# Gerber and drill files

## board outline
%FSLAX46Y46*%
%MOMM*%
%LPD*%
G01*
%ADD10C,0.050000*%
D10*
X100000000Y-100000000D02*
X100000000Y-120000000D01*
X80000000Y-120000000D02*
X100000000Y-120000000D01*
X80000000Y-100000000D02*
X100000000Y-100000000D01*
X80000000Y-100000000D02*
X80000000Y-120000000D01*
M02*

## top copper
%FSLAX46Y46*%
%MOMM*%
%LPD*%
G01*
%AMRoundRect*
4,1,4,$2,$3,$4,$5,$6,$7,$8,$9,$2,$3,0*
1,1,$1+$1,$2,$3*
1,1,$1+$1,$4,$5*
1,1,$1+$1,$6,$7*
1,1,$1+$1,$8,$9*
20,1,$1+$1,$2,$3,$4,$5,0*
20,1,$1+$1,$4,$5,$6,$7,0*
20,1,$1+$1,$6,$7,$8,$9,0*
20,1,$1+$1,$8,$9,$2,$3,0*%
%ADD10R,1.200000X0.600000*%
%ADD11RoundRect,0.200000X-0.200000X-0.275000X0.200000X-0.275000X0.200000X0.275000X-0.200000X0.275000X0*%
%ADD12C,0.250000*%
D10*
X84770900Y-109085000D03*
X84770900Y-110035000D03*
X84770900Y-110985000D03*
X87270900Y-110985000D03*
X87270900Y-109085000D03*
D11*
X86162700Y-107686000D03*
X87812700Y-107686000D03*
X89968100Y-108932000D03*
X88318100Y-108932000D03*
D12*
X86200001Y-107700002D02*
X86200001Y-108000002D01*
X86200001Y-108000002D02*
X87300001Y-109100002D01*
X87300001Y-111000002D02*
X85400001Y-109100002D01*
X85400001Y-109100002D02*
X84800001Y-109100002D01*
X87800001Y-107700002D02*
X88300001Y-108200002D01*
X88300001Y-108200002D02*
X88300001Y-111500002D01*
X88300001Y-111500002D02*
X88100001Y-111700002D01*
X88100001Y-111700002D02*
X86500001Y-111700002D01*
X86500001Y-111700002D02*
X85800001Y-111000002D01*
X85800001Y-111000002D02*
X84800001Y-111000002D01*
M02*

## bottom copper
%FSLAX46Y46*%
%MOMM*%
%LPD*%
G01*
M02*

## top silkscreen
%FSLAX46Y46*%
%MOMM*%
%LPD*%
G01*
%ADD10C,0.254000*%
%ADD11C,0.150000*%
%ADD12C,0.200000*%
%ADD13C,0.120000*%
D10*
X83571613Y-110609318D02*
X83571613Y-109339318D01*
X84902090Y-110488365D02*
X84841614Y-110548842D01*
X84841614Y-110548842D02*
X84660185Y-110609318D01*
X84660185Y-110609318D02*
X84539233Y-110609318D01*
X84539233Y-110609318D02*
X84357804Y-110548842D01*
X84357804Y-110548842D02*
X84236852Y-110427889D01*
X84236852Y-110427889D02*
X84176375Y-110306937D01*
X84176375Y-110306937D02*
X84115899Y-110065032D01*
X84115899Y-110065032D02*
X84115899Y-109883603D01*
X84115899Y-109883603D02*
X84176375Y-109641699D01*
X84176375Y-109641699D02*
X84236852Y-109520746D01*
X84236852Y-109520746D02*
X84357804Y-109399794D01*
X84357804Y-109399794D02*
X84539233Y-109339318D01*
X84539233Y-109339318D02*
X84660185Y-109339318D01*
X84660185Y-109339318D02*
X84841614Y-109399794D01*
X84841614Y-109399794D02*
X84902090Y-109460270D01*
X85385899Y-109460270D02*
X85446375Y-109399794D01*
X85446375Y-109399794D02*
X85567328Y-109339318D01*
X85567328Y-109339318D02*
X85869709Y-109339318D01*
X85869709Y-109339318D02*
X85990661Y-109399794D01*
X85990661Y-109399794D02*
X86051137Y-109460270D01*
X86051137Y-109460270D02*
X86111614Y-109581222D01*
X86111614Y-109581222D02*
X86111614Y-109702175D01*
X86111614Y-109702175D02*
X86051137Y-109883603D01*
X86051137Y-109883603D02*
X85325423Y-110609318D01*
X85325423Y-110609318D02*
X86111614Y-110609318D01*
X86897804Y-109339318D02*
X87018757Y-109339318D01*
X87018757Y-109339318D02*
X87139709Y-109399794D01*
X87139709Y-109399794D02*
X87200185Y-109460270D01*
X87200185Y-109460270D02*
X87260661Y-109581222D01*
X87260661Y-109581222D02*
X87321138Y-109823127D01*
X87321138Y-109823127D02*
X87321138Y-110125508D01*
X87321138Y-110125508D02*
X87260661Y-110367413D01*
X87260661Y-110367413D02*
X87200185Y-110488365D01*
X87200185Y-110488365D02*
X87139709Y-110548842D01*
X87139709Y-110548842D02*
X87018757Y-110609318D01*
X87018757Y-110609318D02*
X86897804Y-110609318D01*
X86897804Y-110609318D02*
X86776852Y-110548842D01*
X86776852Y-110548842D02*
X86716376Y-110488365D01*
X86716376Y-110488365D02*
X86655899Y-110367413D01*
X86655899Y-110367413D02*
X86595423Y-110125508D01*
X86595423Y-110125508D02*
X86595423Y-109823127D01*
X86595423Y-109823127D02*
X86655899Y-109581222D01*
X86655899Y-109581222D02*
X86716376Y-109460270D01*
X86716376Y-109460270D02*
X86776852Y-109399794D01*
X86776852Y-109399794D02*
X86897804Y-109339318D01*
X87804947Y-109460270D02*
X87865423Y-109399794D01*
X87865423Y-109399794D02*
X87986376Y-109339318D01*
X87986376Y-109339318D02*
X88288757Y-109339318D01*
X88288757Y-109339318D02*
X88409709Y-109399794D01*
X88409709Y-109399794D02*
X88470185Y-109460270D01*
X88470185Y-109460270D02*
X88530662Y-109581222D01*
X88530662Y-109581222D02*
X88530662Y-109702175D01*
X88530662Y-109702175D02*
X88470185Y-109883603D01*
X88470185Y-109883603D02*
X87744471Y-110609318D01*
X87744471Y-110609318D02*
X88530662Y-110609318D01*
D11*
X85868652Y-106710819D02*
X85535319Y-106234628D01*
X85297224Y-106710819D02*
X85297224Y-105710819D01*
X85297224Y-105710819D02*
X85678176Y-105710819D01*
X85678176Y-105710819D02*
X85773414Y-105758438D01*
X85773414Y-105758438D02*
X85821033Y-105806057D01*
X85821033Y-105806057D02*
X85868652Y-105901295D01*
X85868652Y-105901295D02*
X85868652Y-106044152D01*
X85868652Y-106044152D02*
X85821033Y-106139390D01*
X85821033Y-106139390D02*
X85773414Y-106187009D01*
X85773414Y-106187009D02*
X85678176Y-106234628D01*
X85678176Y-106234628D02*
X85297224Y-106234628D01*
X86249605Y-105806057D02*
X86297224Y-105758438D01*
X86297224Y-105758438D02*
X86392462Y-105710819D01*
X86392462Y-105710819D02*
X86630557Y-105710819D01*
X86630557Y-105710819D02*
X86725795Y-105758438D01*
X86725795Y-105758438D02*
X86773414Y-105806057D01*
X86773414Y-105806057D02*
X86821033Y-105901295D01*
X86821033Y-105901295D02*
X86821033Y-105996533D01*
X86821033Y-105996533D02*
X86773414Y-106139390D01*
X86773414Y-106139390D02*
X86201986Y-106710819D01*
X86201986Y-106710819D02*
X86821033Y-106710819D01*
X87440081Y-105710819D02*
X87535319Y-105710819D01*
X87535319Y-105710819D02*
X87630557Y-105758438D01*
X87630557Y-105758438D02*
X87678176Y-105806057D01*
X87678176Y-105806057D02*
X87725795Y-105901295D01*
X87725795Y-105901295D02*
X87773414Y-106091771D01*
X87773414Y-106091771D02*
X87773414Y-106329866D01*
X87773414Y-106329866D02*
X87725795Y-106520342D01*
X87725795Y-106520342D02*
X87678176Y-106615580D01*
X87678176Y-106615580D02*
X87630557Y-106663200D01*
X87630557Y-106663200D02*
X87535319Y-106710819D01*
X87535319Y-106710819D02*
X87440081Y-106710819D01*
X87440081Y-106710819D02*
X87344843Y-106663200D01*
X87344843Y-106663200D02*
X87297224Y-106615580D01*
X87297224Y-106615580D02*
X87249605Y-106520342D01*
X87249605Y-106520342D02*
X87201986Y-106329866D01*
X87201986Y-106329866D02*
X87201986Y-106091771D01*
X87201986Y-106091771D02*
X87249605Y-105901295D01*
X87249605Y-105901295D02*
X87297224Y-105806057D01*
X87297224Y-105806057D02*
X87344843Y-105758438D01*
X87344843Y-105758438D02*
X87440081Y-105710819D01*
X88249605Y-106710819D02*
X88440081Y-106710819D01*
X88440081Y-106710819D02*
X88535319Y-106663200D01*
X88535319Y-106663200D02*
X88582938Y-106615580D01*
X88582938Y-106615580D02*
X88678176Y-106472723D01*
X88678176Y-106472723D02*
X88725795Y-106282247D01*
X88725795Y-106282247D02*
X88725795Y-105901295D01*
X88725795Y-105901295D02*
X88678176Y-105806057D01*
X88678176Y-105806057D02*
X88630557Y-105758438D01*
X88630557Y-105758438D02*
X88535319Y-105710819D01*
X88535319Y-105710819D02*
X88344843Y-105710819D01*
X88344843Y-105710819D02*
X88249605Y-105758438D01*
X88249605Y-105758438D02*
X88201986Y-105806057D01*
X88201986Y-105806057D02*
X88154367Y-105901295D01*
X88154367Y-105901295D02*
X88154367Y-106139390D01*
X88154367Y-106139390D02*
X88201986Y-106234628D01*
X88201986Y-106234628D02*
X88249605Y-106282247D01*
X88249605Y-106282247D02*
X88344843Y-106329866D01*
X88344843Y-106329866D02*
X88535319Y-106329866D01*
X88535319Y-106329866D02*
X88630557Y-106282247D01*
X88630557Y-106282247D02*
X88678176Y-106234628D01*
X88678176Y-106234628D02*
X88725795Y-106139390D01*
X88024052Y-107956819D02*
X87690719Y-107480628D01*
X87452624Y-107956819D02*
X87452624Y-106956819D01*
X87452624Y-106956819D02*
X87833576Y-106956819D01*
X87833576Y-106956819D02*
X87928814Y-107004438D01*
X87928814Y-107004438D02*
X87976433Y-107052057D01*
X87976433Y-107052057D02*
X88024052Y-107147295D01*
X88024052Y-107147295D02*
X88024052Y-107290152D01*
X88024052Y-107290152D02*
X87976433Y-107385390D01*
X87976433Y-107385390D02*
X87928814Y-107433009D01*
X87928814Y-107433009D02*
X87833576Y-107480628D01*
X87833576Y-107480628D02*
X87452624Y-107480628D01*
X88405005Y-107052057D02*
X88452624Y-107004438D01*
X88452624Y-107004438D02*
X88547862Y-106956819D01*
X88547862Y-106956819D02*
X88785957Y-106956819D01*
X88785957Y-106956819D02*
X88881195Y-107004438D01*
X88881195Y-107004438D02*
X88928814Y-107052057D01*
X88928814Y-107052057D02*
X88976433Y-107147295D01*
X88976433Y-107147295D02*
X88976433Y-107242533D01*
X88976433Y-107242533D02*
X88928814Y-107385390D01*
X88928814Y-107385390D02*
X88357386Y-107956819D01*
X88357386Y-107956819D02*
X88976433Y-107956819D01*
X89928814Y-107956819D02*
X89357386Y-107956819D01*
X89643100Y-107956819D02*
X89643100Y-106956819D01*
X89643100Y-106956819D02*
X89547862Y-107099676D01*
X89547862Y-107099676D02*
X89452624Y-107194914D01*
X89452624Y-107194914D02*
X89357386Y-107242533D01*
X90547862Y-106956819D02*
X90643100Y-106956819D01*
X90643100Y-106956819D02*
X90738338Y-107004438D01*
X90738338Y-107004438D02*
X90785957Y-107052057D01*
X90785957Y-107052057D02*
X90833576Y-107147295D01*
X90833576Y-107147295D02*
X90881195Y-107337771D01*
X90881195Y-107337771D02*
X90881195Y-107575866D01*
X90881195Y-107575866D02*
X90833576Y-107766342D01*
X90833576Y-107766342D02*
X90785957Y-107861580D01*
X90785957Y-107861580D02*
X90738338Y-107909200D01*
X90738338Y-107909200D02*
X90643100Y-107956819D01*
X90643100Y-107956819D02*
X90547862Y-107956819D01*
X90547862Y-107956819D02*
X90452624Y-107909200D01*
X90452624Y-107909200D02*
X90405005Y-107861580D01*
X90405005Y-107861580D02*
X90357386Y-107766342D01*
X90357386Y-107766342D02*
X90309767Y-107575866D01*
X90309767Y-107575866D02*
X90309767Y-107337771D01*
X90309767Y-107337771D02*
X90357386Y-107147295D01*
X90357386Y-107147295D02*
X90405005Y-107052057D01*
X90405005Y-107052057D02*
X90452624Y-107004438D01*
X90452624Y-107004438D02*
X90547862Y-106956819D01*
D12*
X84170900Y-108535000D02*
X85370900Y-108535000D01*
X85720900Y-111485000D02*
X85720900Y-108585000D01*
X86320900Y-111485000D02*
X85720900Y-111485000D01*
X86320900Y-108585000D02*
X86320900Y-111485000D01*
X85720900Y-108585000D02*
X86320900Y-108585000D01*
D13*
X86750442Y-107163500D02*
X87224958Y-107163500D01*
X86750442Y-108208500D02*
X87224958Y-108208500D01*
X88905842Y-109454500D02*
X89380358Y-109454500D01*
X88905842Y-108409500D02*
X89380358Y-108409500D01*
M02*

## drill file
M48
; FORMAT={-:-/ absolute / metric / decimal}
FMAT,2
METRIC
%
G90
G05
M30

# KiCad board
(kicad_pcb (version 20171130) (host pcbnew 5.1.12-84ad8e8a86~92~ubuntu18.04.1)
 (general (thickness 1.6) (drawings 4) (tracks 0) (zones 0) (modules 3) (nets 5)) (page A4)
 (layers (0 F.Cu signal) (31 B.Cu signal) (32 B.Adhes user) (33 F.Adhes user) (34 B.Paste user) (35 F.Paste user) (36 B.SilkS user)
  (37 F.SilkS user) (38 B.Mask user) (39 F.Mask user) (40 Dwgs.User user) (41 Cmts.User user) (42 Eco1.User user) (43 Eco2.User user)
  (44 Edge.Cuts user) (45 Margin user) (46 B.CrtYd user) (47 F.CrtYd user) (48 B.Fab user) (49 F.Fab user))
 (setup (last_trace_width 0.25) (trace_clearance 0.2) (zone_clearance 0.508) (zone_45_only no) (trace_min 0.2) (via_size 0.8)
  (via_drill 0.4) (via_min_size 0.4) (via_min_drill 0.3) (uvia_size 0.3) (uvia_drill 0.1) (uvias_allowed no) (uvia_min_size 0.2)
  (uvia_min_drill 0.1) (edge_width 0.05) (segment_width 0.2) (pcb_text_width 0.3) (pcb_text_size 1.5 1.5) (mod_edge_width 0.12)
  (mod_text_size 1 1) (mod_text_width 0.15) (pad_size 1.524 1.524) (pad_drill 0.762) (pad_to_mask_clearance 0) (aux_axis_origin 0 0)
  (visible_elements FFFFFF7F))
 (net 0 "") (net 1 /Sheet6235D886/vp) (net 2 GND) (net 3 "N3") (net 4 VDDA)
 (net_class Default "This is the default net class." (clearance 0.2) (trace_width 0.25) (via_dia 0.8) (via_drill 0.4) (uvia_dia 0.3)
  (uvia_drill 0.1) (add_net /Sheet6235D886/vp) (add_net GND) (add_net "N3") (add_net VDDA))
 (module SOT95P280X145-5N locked (layer F.Cu) (at 86.020900 110.035000)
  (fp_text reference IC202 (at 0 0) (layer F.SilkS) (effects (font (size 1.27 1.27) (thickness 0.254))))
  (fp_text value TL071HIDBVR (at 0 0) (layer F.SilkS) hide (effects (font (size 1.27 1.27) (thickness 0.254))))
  (fp_line (start -1.85 -1.5) (end -0.65 -1.5) (layer F.SilkS) (width 0.2))
  (fp_line (start -0.3 1.45) (end -0.3 -1.45) (layer F.SilkS) (width 0.2))
  (fp_line (start 0.3 1.45) (end -0.3 1.45) (layer F.SilkS) (width 0.2))
  (fp_line (start 0.3 -1.45) (end 0.3 1.45) (layer F.SilkS) (width 0.2))
  (fp_line (start -0.3 -1.45) (end 0.3 -1.45) (layer F.SilkS) (width 0.2))
  (pad 1 smd rect (at -1.25 -0.95 90.000000) (size 0.6 1.2) (layers F.Cu F.Mask F.Paste) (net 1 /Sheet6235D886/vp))
  (pad 2 smd rect (at -1.25 0 90.000000) (size 0.6 1.2) (layers F.Cu F.Mask F.Paste) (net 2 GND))
  (pad 3 smd rect (at -1.25 0.95 90.000000) (size 0.6 1.2) (layers F.Cu F.Mask F.Paste) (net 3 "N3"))
  (pad 4 smd rect (at 1.25 0.95 90.000000) (size 0.6 1.2) (layers F.Cu F.Mask F.Paste) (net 1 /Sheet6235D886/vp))
  (pad 5 smd rect (at 1.25 -0.95 90.000000) (size 0.6 1.2) (layers F.Cu F.Mask F.Paste) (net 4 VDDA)))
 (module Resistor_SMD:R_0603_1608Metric (layer F.Cu) (at 86.987700 107.686000)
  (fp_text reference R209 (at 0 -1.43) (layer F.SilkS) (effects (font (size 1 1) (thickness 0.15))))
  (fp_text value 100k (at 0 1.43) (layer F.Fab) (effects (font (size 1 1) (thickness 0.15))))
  (fp_line (start -0.237258 -0.5225) (end 0.237258 -0.5225) (layer F.SilkS) (width 0.12))
  (fp_line (start -0.237258 0.5225) (end 0.237258 0.5225) (layer F.SilkS) (width 0.12))
  (pad 1 smd roundrect (at -0.825 0) (size 0.8 0.95) (layers F.Cu F.Mask F.Paste) (roundrect_rratio 0.25) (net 4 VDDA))
  (pad 2 smd roundrect (at 0.825 0) (size 0.8 0.95) (layers F.Cu F.Mask F.Paste) (roundrect_rratio 0.25) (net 3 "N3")))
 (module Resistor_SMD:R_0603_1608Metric (layer F.Cu) (at 89.143100 108.932000)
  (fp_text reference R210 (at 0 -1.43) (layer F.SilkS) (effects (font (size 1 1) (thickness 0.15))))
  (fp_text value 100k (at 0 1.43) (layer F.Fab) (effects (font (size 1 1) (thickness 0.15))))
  (fp_line (start -0.237258 0.5225) (end 0.237258 0.5225) (layer F.SilkS) (width 0.12))
  (fp_line (start -0.237258 -0.5225) (end 0.237258 -0.5225) (layer F.SilkS) (width 0.12))
  (pad 2 smd roundrect (at 0.825 0) (size 0.8 0.95) (layers F.Cu F.Mask F.Paste) (roundrect_rratio 0.25) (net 2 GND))
  (pad 1 smd roundrect (at -0.825 0) (size 0.8 0.95) (layers F.Cu F.Mask F.Paste) (roundrect_rratio 0.25) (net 3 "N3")))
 (gr_line (start 100 100) (end 100 120) (layer Edge.Cuts) (width 0.05))
 (gr_line (start 80 120) (end 100 120) (layer Edge.Cuts) (width 0.05))
 (gr_line (start 80 100) (end 100 100) (layer Edge.Cuts) (width 0.05))
 (gr_line (start 80 100) (end 80 120) (layer Edge.Cuts) (width 0.05))
 (segment (start 86.200001 107.700002) (end 86.200001 108.000002) (width 0.250000) (layer F.Cu) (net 4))
 (segment (start 86.200001 108.000002) (end 87.300001 109.100002) (width 0.250000) (layer F.Cu) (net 4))
 (segment (start 87.300001 111.000002) (end 85.400001 109.100002) (width 0.250000) (layer F.Cu) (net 1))
 (segment (start 85.400001 109.100002) (end 84.800001 109.100002) (width 0.250000) (layer F.Cu) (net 1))
 (segment (start 87.800001 107.700002) (end 88.300001 108.200002) (width 0.250000) (layer F.Cu) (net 3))
 (segment (start 88.300001 108.200002) (end 88.300001 111.500002) (width 0.250000) (layer F.Cu) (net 3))
 (segment (start 88.300001 111.500002) (end 88.100001 111.700002) (width 0.250000) (layer F.Cu) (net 3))
 (segment (start 88.100001 111.700002) (end 86.500001 111.700002) (width 0.250000) (layer F.Cu) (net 3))
 (segment (start 86.500001 111.700002) (end 85.800001 111.000002) (width 0.250000) (layer F.Cu) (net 3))
 (segment (start 85.800001 111.000002) (end 84.800001 111.000002) (width 0.250000) (layer F.Cu) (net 3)))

